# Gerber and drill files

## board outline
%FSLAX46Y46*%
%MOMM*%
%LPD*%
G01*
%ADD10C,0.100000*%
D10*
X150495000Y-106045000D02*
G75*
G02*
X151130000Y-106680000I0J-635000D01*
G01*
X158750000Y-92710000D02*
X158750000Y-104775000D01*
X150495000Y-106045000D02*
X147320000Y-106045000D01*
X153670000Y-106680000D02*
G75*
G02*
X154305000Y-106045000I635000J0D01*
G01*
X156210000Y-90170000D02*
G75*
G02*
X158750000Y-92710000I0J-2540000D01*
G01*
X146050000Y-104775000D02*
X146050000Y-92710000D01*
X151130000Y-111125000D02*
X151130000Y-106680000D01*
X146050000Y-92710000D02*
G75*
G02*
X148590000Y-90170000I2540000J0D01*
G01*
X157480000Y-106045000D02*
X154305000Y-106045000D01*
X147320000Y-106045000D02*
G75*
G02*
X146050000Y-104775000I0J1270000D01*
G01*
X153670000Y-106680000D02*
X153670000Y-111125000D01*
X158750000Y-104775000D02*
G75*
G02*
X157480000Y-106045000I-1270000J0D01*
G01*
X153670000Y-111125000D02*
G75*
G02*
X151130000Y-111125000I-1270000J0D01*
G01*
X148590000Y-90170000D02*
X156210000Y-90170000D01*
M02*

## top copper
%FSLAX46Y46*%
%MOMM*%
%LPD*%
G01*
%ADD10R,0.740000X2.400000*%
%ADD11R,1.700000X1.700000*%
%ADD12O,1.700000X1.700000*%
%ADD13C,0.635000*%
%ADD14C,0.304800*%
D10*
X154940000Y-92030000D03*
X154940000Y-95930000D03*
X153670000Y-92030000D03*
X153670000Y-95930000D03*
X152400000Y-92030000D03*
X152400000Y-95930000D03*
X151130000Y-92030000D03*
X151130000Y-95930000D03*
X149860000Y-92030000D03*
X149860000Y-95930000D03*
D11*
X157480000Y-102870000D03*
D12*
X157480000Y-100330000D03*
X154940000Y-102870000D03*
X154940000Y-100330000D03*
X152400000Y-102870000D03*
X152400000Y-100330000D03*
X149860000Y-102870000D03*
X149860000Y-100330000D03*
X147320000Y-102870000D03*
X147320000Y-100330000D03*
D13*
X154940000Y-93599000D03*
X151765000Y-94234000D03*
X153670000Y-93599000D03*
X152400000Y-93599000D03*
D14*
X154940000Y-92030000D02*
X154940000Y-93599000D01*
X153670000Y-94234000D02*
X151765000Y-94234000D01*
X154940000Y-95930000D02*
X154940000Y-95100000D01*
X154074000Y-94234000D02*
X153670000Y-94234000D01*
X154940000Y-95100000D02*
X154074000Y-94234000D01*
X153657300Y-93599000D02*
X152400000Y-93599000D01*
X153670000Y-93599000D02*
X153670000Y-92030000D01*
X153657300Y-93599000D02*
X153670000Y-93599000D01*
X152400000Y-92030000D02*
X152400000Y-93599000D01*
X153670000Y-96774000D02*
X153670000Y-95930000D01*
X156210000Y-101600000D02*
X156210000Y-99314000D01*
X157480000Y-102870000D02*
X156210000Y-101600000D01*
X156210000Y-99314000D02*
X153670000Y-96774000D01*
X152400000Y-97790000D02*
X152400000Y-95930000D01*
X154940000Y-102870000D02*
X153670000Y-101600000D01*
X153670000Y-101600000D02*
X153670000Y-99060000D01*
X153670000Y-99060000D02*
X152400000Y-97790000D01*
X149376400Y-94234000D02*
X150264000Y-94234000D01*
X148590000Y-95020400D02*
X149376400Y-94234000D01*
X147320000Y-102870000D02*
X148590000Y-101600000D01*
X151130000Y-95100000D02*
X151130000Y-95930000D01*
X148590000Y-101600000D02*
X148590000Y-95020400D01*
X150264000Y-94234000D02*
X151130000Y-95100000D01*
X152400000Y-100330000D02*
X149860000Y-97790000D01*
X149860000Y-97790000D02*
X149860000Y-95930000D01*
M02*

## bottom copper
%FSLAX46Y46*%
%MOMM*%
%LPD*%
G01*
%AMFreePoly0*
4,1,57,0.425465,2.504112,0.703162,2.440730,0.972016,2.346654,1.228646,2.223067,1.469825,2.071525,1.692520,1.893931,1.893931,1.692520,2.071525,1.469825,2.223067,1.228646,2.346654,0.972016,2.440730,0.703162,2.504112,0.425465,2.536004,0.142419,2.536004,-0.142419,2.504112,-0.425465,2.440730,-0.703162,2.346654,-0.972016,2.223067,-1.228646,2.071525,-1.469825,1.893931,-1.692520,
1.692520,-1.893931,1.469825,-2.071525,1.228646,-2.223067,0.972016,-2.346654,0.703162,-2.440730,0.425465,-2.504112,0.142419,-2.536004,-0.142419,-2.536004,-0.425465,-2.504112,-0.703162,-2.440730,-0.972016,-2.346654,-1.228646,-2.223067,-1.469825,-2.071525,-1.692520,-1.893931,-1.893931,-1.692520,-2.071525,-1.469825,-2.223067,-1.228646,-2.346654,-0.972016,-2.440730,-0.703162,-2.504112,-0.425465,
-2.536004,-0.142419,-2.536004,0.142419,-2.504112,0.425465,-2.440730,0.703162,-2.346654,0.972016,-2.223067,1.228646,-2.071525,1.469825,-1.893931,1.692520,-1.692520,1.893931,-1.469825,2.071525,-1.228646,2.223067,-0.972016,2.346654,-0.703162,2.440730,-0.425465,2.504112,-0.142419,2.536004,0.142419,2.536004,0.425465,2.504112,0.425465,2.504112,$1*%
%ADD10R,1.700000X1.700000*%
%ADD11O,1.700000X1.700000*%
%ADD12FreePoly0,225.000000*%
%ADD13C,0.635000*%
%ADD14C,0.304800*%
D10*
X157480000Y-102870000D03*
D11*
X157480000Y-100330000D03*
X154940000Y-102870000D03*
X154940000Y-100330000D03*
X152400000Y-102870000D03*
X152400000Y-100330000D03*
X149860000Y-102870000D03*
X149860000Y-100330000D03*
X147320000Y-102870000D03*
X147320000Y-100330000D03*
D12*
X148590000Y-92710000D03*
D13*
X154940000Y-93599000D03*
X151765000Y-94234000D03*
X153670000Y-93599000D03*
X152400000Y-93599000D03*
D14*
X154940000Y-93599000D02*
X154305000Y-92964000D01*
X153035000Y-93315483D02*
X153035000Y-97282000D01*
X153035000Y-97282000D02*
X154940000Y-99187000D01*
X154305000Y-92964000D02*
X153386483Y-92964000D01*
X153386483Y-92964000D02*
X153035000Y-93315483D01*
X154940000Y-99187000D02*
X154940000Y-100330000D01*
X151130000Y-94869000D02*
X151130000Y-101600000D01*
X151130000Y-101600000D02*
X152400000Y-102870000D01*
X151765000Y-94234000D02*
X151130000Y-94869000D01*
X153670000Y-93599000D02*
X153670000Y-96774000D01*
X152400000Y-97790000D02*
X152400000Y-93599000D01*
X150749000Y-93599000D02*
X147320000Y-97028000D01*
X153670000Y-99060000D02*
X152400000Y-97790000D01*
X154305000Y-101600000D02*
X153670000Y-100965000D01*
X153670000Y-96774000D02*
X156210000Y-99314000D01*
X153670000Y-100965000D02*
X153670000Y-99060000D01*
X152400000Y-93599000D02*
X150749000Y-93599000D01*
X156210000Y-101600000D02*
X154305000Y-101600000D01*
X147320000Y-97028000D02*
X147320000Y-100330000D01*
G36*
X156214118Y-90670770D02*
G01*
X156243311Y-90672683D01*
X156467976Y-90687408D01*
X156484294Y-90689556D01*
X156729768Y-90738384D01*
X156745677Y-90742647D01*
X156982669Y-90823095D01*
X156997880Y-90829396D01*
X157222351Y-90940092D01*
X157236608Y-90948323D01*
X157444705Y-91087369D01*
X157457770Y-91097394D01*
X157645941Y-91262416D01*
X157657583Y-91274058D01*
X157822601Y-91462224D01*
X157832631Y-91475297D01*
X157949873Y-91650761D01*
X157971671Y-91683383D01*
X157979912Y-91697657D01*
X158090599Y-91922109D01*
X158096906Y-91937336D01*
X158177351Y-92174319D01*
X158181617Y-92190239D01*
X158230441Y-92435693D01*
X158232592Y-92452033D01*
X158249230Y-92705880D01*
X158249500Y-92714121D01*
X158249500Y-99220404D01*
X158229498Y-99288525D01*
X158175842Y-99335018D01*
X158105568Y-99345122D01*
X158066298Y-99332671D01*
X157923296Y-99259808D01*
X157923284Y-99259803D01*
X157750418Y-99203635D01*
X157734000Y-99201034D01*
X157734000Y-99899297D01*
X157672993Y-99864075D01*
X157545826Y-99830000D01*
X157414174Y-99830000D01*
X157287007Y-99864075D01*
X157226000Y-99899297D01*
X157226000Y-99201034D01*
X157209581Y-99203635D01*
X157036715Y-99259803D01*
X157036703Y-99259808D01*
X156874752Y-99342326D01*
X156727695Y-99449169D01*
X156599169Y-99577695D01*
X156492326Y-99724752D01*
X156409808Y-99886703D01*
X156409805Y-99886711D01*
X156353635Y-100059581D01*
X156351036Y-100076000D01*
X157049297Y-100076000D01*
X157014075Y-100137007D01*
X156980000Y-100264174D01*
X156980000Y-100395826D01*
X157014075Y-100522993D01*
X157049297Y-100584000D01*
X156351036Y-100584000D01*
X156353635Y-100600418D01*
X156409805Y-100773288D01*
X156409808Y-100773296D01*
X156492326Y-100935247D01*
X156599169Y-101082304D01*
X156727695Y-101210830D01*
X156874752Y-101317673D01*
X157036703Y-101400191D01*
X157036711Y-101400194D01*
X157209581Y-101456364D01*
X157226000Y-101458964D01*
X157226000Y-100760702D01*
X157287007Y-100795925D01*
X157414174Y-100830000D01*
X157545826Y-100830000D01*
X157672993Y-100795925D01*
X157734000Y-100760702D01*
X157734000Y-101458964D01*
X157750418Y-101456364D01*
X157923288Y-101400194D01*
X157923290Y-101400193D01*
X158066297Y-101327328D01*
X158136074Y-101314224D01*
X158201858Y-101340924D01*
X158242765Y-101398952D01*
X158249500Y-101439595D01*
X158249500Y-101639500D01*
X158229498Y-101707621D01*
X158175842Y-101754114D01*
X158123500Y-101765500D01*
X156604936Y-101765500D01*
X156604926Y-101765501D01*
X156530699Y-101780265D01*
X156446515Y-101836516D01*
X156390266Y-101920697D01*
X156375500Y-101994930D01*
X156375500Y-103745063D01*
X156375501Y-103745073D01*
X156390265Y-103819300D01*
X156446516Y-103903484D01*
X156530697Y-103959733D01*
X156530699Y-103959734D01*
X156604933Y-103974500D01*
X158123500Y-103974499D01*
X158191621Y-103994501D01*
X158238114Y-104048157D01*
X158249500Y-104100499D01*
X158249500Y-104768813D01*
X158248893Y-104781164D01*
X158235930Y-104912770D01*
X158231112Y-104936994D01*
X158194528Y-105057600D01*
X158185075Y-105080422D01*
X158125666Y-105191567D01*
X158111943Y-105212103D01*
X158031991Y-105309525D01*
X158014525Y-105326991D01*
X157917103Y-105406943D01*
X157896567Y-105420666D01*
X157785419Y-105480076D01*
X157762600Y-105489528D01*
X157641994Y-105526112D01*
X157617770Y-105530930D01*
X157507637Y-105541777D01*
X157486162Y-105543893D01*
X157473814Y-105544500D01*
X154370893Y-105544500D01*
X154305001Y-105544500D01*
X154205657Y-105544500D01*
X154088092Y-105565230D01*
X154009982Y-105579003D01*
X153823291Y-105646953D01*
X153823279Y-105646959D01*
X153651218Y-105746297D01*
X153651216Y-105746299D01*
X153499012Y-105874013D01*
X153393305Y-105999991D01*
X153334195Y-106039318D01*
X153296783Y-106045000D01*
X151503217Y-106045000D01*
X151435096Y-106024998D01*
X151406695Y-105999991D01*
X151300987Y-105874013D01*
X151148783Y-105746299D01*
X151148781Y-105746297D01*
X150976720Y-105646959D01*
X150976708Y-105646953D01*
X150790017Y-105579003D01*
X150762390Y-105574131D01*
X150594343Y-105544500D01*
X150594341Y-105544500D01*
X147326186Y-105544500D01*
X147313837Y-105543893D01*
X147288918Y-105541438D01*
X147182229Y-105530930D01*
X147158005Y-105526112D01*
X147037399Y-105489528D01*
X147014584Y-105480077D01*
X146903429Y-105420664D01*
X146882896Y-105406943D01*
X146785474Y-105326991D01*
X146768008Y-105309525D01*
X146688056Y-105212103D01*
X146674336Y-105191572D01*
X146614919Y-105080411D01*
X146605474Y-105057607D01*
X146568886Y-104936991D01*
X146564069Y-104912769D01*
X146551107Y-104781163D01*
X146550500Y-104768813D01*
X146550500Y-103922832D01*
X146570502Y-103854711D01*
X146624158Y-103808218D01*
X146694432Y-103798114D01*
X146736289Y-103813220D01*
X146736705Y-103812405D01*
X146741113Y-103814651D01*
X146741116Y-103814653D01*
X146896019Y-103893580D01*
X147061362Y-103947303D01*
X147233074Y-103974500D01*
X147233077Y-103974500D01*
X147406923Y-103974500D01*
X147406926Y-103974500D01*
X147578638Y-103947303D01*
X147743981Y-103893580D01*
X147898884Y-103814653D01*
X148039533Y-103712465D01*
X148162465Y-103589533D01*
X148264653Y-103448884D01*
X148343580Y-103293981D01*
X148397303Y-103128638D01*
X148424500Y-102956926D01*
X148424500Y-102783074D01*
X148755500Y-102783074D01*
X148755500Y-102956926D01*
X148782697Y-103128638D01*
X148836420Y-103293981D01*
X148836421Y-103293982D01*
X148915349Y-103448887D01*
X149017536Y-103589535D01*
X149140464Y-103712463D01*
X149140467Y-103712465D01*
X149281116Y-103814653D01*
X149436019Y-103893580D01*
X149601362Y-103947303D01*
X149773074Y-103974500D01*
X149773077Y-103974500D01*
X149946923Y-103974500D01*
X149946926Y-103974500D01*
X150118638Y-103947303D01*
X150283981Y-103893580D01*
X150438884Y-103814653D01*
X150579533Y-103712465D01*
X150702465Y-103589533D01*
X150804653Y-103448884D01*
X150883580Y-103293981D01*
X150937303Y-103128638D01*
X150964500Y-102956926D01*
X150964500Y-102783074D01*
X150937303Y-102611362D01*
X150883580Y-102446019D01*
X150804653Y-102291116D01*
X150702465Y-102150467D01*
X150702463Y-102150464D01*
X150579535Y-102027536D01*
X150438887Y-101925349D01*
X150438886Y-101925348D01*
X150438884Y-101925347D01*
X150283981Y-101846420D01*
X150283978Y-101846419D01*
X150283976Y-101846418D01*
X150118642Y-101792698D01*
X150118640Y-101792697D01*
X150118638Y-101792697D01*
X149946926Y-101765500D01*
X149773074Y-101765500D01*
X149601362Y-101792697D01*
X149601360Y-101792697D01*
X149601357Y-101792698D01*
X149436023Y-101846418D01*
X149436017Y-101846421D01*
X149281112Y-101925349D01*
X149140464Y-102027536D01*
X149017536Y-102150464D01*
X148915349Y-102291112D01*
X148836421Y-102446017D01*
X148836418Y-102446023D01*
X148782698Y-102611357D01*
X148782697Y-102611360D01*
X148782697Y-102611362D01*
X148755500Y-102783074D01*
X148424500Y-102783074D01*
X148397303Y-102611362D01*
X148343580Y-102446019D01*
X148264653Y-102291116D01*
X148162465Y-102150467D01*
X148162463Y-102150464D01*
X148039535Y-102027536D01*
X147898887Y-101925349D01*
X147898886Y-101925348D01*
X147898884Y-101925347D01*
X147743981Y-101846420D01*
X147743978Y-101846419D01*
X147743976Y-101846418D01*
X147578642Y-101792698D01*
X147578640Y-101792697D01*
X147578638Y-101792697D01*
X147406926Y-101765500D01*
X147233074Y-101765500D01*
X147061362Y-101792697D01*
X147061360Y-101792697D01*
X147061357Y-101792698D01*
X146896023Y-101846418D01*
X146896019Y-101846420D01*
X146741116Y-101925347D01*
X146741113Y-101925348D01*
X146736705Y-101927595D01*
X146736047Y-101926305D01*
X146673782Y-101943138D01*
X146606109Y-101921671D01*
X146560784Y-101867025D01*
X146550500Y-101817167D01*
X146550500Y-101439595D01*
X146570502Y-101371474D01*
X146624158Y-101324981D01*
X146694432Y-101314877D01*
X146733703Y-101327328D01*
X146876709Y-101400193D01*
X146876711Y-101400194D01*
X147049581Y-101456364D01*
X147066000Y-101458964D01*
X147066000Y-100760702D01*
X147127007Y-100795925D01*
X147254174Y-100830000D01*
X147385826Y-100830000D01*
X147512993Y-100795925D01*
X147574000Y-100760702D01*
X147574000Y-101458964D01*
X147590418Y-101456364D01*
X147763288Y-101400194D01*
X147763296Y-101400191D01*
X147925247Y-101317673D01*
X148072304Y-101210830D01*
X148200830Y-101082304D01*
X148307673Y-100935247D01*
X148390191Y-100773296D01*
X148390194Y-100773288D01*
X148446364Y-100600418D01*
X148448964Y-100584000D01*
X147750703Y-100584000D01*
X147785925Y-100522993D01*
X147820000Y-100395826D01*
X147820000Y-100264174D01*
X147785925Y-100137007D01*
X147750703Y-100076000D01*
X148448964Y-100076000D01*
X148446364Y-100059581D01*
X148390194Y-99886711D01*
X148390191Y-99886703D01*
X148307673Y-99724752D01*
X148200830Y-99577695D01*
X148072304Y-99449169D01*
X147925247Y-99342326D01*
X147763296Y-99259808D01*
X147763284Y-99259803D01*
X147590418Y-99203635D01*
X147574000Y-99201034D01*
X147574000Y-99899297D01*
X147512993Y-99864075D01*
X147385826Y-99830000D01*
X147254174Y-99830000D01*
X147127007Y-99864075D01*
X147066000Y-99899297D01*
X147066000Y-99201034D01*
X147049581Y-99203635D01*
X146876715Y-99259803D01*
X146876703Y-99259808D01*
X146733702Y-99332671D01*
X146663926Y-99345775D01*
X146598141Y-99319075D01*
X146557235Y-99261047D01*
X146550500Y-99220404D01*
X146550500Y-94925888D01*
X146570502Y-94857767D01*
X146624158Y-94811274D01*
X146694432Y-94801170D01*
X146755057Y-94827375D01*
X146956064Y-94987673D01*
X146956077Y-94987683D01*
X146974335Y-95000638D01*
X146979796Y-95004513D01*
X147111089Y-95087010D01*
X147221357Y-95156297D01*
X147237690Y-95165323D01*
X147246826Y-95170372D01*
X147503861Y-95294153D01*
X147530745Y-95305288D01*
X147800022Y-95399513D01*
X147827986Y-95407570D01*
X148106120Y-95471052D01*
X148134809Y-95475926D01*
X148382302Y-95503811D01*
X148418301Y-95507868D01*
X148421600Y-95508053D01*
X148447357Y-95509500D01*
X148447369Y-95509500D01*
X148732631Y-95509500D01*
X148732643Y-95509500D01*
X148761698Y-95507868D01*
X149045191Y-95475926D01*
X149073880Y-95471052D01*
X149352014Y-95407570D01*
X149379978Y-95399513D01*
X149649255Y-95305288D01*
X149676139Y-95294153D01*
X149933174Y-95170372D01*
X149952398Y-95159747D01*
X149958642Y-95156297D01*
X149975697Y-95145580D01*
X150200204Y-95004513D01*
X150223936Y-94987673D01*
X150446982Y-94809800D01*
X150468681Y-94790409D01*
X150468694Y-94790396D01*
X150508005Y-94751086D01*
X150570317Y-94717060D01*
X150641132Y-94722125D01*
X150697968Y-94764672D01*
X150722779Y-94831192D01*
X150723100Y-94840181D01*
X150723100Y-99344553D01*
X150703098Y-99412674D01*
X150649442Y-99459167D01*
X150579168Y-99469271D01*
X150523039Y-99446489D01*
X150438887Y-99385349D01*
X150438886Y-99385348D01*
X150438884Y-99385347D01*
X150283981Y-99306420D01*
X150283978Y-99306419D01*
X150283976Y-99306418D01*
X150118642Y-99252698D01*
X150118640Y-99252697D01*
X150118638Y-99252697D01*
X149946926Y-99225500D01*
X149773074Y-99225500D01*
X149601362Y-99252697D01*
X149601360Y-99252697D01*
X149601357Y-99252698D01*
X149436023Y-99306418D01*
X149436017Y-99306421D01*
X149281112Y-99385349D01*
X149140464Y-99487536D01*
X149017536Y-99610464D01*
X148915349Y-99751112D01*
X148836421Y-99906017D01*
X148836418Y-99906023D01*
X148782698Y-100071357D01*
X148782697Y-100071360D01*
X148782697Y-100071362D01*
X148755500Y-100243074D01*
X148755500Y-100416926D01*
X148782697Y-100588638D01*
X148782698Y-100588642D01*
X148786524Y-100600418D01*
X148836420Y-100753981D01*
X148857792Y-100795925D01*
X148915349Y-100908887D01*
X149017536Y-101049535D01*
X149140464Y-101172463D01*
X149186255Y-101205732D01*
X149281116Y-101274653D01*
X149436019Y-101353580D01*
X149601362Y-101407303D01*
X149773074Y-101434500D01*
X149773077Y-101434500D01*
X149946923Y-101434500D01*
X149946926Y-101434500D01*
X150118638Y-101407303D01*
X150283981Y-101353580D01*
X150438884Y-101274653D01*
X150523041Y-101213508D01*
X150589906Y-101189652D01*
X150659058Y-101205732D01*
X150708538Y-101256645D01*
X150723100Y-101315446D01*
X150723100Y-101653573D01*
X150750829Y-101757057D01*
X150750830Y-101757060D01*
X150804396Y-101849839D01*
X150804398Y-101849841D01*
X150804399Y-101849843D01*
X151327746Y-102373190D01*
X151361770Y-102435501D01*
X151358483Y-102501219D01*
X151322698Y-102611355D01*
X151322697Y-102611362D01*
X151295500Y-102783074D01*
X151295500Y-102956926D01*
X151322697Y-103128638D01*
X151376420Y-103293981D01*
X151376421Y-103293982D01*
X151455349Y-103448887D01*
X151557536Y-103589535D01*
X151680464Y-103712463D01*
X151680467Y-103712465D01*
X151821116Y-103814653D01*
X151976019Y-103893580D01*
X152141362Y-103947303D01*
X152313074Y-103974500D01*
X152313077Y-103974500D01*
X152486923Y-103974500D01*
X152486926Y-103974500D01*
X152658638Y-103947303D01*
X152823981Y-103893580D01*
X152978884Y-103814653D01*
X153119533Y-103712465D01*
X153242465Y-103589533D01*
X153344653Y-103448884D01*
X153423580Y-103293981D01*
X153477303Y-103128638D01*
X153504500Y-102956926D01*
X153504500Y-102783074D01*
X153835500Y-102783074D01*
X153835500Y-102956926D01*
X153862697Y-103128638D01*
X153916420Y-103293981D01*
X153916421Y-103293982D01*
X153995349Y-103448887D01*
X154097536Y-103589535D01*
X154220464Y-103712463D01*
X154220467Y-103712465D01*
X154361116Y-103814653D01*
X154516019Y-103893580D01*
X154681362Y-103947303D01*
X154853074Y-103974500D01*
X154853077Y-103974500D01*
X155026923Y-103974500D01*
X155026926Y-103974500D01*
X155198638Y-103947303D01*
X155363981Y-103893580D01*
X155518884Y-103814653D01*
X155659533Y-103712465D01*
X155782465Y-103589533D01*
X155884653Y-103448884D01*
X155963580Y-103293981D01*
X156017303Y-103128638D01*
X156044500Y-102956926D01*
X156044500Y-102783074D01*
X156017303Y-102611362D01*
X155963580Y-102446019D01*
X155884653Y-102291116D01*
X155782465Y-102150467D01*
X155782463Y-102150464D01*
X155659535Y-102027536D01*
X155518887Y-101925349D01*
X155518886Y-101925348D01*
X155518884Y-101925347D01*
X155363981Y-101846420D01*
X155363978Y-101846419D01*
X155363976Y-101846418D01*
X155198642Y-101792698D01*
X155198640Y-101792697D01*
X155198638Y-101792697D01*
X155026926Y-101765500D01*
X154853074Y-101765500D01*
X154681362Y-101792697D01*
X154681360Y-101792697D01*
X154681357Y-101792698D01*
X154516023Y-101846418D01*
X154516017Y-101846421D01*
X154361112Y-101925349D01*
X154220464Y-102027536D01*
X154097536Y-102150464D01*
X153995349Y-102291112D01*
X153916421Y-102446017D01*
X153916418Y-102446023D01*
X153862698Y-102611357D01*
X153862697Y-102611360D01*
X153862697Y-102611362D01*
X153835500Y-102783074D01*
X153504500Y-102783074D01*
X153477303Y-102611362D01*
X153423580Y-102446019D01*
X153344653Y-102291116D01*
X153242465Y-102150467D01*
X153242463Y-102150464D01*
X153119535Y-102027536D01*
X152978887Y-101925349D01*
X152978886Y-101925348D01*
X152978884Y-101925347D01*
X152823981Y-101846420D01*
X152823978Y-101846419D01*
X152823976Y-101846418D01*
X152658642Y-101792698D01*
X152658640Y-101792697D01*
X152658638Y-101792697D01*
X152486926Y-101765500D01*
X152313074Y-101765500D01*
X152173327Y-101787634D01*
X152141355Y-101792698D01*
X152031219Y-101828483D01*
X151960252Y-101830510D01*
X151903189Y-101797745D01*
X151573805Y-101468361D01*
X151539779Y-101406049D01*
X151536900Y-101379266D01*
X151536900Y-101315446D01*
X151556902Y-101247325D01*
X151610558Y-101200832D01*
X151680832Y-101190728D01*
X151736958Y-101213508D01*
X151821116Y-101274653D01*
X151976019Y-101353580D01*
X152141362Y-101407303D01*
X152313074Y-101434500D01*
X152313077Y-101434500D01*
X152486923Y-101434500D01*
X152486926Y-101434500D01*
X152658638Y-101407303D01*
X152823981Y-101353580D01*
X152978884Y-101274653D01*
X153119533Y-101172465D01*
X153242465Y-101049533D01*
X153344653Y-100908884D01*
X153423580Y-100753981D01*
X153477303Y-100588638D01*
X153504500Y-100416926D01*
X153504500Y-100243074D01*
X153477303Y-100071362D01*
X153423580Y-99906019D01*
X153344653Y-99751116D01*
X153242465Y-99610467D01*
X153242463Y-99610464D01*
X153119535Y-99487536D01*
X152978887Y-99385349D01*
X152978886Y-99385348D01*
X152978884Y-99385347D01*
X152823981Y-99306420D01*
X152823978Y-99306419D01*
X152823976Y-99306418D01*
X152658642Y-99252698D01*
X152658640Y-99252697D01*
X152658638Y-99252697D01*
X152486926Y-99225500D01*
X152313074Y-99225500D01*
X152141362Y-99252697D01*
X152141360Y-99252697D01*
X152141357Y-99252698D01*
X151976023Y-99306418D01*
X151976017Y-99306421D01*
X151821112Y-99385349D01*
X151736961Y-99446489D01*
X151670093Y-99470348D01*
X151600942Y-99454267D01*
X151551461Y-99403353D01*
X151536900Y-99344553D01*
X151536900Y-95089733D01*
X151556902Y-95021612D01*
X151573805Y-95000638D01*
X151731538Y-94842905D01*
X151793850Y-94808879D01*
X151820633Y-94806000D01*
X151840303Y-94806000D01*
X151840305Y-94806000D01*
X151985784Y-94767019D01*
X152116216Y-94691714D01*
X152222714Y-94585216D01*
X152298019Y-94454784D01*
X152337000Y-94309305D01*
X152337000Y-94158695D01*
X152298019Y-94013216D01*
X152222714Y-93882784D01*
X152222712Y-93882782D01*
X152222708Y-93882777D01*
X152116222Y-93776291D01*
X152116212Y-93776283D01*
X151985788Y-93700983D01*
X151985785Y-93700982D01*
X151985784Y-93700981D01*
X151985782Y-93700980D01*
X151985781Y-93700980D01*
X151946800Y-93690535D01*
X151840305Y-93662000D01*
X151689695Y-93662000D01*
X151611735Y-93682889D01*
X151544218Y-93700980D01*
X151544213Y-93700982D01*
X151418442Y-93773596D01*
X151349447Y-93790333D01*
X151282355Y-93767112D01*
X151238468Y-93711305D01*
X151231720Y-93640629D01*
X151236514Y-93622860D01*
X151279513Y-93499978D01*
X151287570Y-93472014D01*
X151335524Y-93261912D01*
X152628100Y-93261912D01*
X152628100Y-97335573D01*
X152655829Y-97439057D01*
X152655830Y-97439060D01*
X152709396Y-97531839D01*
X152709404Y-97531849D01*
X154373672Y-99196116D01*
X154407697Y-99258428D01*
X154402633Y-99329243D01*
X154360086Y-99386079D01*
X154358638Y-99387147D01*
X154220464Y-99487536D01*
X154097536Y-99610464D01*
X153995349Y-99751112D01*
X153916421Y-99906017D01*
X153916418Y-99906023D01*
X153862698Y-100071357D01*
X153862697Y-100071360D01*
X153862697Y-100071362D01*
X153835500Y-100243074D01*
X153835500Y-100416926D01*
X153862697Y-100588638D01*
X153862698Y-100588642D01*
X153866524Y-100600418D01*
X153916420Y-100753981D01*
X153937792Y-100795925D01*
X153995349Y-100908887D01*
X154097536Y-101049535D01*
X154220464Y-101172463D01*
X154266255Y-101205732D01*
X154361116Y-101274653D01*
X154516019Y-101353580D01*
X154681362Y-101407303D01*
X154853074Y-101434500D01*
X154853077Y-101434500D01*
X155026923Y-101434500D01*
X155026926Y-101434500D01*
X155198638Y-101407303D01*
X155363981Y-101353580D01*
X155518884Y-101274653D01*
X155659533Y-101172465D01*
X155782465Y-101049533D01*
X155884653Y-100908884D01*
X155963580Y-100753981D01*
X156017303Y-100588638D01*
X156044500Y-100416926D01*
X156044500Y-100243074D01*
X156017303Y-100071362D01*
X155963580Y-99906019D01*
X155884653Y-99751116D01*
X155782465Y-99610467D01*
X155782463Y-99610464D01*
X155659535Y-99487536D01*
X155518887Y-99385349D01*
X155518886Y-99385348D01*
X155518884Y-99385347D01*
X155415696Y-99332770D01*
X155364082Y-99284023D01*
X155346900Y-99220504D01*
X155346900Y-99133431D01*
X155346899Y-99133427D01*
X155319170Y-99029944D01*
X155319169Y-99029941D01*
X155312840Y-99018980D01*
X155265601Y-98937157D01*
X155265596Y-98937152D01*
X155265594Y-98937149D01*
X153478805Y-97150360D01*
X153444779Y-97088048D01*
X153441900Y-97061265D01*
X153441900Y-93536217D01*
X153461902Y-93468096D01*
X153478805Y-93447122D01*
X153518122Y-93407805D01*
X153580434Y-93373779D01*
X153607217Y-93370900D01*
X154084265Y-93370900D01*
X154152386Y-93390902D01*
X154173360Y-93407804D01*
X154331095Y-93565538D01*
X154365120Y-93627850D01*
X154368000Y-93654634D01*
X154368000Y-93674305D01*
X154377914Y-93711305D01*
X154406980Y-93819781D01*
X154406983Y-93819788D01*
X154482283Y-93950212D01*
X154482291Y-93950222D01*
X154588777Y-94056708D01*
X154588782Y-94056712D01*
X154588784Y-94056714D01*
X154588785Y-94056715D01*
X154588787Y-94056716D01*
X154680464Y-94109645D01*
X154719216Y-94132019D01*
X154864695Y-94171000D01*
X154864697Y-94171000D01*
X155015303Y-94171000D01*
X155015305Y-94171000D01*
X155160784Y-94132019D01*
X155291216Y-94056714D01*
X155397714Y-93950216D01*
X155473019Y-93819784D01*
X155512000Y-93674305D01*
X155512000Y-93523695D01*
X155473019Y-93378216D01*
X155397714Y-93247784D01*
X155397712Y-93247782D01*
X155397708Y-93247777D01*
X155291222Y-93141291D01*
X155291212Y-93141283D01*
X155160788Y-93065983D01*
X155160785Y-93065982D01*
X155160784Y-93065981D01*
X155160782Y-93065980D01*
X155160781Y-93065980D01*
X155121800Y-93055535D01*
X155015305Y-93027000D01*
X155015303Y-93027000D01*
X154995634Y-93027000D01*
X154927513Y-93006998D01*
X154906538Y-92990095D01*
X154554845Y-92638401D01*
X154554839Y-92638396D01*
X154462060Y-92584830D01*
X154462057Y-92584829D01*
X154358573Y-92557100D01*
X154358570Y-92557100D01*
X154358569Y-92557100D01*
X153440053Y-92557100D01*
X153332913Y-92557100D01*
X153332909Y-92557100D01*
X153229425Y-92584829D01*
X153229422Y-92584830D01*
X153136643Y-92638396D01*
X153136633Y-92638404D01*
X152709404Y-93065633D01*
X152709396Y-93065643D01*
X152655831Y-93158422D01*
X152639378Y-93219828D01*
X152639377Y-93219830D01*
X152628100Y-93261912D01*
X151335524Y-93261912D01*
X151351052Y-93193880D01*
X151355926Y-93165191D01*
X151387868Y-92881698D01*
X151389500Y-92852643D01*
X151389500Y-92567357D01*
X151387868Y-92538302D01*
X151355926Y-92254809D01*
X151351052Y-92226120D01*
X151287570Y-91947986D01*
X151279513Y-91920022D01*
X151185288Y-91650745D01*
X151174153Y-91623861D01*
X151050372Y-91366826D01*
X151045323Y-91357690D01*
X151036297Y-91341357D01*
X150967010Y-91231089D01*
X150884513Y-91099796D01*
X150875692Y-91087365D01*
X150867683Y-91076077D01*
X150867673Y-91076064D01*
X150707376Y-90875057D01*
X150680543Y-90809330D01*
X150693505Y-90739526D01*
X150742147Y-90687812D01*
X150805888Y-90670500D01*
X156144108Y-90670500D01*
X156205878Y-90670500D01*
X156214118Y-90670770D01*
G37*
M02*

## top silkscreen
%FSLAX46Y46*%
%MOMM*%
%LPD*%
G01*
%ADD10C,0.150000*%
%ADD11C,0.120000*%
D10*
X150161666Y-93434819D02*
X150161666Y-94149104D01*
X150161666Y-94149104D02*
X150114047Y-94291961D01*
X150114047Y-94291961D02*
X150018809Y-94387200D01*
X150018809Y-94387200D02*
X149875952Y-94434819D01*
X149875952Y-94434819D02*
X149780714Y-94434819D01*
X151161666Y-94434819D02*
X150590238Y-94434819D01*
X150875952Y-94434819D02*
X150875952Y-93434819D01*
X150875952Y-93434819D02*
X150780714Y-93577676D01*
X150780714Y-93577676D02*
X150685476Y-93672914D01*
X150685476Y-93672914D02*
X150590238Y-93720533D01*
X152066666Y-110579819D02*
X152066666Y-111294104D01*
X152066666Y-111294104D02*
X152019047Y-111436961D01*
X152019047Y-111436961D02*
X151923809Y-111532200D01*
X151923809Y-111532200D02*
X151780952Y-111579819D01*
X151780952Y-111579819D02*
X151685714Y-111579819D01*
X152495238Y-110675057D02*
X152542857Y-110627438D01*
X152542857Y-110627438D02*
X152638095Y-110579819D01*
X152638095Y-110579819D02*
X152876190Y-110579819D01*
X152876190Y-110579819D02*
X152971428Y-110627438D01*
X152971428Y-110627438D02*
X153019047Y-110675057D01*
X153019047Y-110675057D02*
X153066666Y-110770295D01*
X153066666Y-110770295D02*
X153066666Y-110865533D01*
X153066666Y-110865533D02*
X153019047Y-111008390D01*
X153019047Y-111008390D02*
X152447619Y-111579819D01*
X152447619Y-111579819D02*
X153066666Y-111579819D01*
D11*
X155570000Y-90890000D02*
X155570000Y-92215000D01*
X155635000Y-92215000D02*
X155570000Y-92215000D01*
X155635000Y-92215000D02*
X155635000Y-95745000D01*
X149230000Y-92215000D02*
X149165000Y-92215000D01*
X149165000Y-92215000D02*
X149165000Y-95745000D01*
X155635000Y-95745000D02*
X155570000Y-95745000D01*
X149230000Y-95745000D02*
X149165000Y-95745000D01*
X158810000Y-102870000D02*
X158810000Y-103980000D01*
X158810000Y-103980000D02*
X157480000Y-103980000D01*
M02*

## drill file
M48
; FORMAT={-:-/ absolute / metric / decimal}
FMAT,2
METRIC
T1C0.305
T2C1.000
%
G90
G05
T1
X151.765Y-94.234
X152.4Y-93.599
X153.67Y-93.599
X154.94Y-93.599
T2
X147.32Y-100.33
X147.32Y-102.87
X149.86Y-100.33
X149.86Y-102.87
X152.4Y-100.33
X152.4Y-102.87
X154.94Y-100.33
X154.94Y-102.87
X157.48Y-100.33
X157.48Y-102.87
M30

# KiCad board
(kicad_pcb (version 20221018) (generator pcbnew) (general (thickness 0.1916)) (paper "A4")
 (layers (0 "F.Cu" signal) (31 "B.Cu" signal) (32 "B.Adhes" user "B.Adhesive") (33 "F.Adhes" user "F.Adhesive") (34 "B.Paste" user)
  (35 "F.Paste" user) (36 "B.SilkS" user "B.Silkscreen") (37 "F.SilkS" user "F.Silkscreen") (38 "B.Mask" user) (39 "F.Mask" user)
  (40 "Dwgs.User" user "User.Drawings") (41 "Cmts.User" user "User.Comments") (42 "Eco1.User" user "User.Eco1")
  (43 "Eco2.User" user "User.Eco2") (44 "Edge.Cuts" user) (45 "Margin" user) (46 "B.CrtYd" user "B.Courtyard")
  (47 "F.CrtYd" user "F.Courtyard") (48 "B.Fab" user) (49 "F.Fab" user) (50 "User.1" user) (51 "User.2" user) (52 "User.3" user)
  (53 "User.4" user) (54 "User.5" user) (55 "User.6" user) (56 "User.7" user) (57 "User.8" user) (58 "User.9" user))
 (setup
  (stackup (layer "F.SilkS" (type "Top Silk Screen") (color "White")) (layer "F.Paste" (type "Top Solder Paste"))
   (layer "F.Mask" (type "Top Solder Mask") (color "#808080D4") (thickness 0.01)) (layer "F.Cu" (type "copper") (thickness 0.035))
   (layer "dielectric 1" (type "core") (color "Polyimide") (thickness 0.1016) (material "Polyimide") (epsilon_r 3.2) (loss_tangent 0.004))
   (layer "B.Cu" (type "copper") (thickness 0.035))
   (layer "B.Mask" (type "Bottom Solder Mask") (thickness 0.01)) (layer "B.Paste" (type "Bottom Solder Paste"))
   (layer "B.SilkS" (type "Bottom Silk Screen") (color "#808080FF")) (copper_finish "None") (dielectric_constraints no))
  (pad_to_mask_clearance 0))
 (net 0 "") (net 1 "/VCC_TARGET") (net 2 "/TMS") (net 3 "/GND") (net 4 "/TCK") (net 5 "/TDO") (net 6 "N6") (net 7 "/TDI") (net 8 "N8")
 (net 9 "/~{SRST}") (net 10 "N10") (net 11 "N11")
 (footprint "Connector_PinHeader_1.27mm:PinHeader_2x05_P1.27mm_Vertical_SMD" (layer "F.Cu") (at 152.4 93.98 -90)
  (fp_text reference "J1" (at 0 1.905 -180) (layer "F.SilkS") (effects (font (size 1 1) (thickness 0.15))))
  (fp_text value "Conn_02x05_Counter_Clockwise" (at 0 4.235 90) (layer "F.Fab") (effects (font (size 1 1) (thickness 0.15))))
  (fp_line (start -3.09 -3.17) (end -1.765 -3.17) (stroke (width 0.12) (type solid)) (layer "F.SilkS"))
  (fp_line (start -1.765 -3.235) (end -1.765 -3.17) (stroke (width 0.12) (type solid)) (layer "F.SilkS"))
  (fp_line (start -1.765 -3.235) (end 1.765 -3.235) (stroke (width 0.12) (type solid)) (layer "F.SilkS"))
  (fp_line (start -1.765 3.17) (end -1.765 3.235) (stroke (width 0.12) (type solid)) (layer "F.SilkS"))
  (fp_line (start -1.765 3.235) (end 1.765 3.235) (stroke (width 0.12) (type solid)) (layer "F.SilkS"))
  (fp_line (start 1.765 -3.235) (end 1.765 -3.17) (stroke (width 0.12) (type solid)) (layer "F.SilkS"))
  (fp_line (start 1.765 3.17) (end 1.765 3.235) (stroke (width 0.12) (type solid)) (layer "F.SilkS"))
  (pad "1" smd rect (at -1.95 -2.54 270) (size 2.4 0.74) (layers "F.Cu" "F.Paste" "F.Mask") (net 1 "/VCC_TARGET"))
  (pad "2" smd rect (at 1.95 -2.54 270) (size 2.4 0.74) (layers "F.Cu" "F.Paste" "F.Mask") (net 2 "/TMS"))
  (pad "3" smd rect (at -1.95 -1.27 270) (size 2.4 0.74) (layers "F.Cu" "F.Paste" "F.Mask") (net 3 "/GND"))
  (pad "4" smd rect (at 1.95 -1.27 270) (size 2.4 0.74) (layers "F.Cu" "F.Paste" "F.Mask") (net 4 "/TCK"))
  (pad "5" smd rect (at -1.95 0 270) (size 2.4 0.74) (layers "F.Cu" "F.Paste" "F.Mask") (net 3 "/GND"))
  (pad "6" smd rect (at 1.95 0 270) (size 2.4 0.74) (layers "F.Cu" "F.Paste" "F.Mask") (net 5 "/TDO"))
  (pad "7" smd rect (at -1.95 1.27 270) (size 2.4 0.74) (layers "F.Cu" "F.Paste" "F.Mask") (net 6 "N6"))
  (pad "8" smd rect (at 1.95 1.27 270) (size 2.4 0.74) (layers "F.Cu" "F.Paste" "F.Mask") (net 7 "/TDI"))
  (pad "9" smd rect (at -1.95 2.54 270) (size 2.4 0.74) (layers "F.Cu" "F.Paste" "F.Mask") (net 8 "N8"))
  (pad "10" smd rect (at 1.95 2.54 270) (size 2.4 0.74) (layers "F.Cu" "F.Paste" "F.Mask") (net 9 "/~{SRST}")))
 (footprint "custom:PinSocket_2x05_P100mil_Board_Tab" (layer "F.Cu") (at 157.48 102.87 -90)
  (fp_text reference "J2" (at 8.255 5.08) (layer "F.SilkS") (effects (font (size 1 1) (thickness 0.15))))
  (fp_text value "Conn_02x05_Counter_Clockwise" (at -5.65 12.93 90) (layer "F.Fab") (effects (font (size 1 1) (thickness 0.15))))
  (fp_line (start 0 -1.33) (end 1.11 -1.33) (stroke (width 0.12) (type solid)) (layer "F.SilkS"))
  (fp_line (start 1.11 -1.33) (end 1.11 0) (stroke (width 0.12) (type solid)) (layer "F.SilkS"))
  (pad "1" thru_hole rect (at 0 0 270) (size 1.7 1.7) (drill 1) (layers "*.Cu" "*.Mask") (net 4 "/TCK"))
  (pad "2" thru_hole oval (at -2.54 0 270) (size 1.7 1.7) (drill 1) (layers "*.Cu" "*.Mask") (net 3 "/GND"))
  (pad "3" thru_hole oval (at 0 2.54 270) (size 1.7 1.7) (drill 1) (layers "*.Cu" "*.Mask") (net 5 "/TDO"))
  (pad "4" thru_hole oval (at -2.54 2.54 270) (size 1.7 1.7) (drill 1) (layers "*.Cu" "*.Mask") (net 1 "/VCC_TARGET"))
  (pad "5" thru_hole oval (at 0 5.08 270) (size 1.7 1.7) (drill 1) (layers "*.Cu" "*.Mask") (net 2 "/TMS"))
  (pad "6" thru_hole oval (at -2.54 5.08 270) (size 1.7 1.7) (drill 1) (layers "*.Cu" "*.Mask") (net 9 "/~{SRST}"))
  (pad "7" thru_hole oval (at 0 7.62 270) (size 1.7 1.7) (drill 1) (layers "*.Cu" "*.Mask") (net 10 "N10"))
  (pad "8" thru_hole oval (at -2.54 7.62 270) (size 1.7 1.7) (drill 1) (layers "*.Cu" "*.Mask") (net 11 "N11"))
  (pad "9" thru_hole oval (at 0 10.16 270) (size 1.7 1.7) (drill 1) (layers "*.Cu" "*.Mask") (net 7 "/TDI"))
  (pad "10" thru_hole oval (at -2.54 10.16 270) (size 1.7 1.7) (drill 1) (layers "*.Cu" "*.Mask") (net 3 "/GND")))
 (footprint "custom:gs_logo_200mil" (layer "B.Cu") (at 148.59 92.71 -135)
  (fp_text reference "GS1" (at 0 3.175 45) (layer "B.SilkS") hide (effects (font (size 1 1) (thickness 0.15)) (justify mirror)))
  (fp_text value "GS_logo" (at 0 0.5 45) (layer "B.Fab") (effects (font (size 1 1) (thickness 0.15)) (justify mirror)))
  (pad "1" smd custom (at 0 0 225) (size 5.08 5.08) (layers "B.Cu") (zone_connect 0) (options (clearance outline) (anchor circle))
   (primitives)))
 (gr_arc (start 150.495 106.045) (mid 150.944013 106.230987) (end 151.13 106.68) (stroke (width 0.1) (type default)) (layer "Edge.Cuts"))
 (gr_line (start 158.75 92.71) (end 158.75 104.775) (stroke (width 0.1) (type default)) (layer "Edge.Cuts"))
 (gr_line (start 150.495 106.045) (end 147.32 106.045) (stroke (width 0.1) (type default)) (layer "Edge.Cuts"))
 (gr_arc (start 153.67 106.68) (mid 153.855987 106.230987) (end 154.305 106.045) (stroke (width 0.1) (type default)) (layer "Edge.Cuts"))
 (gr_arc (start 156.21 90.17) (mid 158.006051 90.913949) (end 158.75 92.71) (stroke (width 0.1) (type default)) (layer "Edge.Cuts"))
 (gr_line (start 146.05 104.775) (end 146.05 92.71) (stroke (width 0.1) (type default)) (layer "Edge.Cuts"))
 (gr_line (start 151.13 111.125) (end 151.13 106.68) (stroke (width 0.1) (type default)) (layer "Edge.Cuts"))
 (gr_arc (start 146.05 92.71) (mid 146.793949 90.913949) (end 148.59 90.17) (stroke (width 0.1) (type default)) (layer "Edge.Cuts"))
 (gr_line (start 157.48 106.045) (end 154.305 106.045) (stroke (width 0.1) (type default)) (layer "Edge.Cuts"))
 (gr_arc (start 147.32 106.045) (mid 146.421974 105.673026) (end 146.05 104.775) (stroke (width 0.1) (type default)) (layer "Edge.Cuts"))
 (gr_line (start 153.67 106.68) (end 153.67 111.125) (stroke (width 0.1) (type default)) (layer "Edge.Cuts"))
 (gr_arc (start 158.75 104.775) (mid 158.378026 105.673026) (end 157.48 106.045) (stroke (width 0.1) (type default)) (layer "Edge.Cuts"))
 (gr_arc (start 153.67 111.125) (mid 152.4 112.395) (end 151.13 111.125) (stroke (width 0.1) (type default)) (layer "Edge.Cuts"))
 (gr_line (start 148.59 90.17) (end 156.21 90.17) (stroke (width 0.1) (type default)) (layer "Edge.Cuts"))
 (segment (start 154.94 92.03) (end 154.94 93.599) (width 0.3048) (layer "F.Cu") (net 1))
 (via (at 154.94 93.599) (size 0.635) (drill 0.3048) (layers "F.Cu" "B.Cu") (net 1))
 (segment (start 154.94 93.599) (end 154.305 92.964) (width 0.3048) (layer "B.Cu") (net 1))
 (segment (start 153.035 93.315483) (end 153.035 97.282) (width 0.3048) (layer "B.Cu") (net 1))
 (segment (start 153.035 97.282) (end 154.94 99.187) (width 0.3048) (layer "B.Cu") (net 1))
 (segment (start 154.305 92.964) (end 153.386483 92.964) (width 0.3048) (layer "B.Cu") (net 1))
 (segment (start 153.386483 92.964) (end 153.035 93.315483) (width 0.3048) (layer "B.Cu") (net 1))
 (segment (start 154.94 99.187) (end 154.94 100.33) (width 0.3048) (layer "B.Cu") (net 1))
 (segment (start 153.67 94.234) (end 151.765 94.234) (width 0.3048) (layer "F.Cu") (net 2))
 (segment (start 154.94 95.93) (end 154.94 95.1) (width 0.3048) (layer "F.Cu") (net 2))
 (segment (start 154.074 94.234) (end 153.67 94.234) (width 0.3048) (layer "F.Cu") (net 2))
 (segment (start 154.94 95.1) (end 154.074 94.234) (width 0.3048) (layer "F.Cu") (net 2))
 (via (at 151.765 94.234) (size 0.635) (drill 0.3048) (layers "F.Cu" "B.Cu") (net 2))
 (segment (start 151.13 94.869) (end 151.13 101.6) (width 0.3048) (layer "B.Cu") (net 2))
 (segment (start 151.13 101.6) (end 152.4 102.87) (width 0.3048) (layer "B.Cu") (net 2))
 (segment (start 151.765 94.234) (end 151.13 94.869) (width 0.3048) (layer "B.Cu") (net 2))
 (segment (start 153.6573 93.599) (end 152.4 93.599) (width 0.3048) (layer "F.Cu") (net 3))
 (segment (start 153.67 93.599) (end 153.67 92.03) (width 0.3048) (layer "F.Cu") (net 3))
 (segment (start 153.6573 93.599) (end 153.67 93.599) (width 0.3048) (layer "F.Cu") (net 3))
 (segment (start 152.4 92.03) (end 152.4 93.599) (width 0.3048) (layer "F.Cu") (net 3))
 (via (at 153.67 93.599) (size 0.635) (drill 0.3048) (layers "F.Cu" "B.Cu") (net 3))
 (via (at 152.4 93.599) (size 0.635) (drill 0.3048) (layers "F.Cu" "B.Cu") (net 3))
 (segment (start 153.67 93.599) (end 153.67 96.774) (width 0.3048) (layer "B.Cu") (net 3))
 (segment (start 152.4 97.79) (end 152.4 93.599) (width 0.3048) (layer "B.Cu") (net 3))
 (segment (start 150.749 93.599) (end 147.32 97.028) (width 0.3048) (layer "B.Cu") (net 3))
 (segment (start 153.67 99.06) (end 152.4 97.79) (width 0.3048) (layer "B.Cu") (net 3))
 (segment (start 154.305 101.6) (end 153.67 100.965) (width 0.3048) (layer "B.Cu") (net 3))
 (segment (start 153.67 96.774) (end 156.21 99.314) (width 0.3048) (layer "B.Cu") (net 3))
 (segment (start 153.67 100.965) (end 153.67 99.06) (width 0.3048) (layer "B.Cu") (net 3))
 (segment (start 152.4 93.599) (end 150.749 93.599) (width 0.3048) (layer "B.Cu") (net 3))
 (segment (start 156.21 101.6) (end 154.305 101.6) (width 0.3048) (layer "B.Cu") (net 3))
 (segment (start 147.32 97.028) (end 147.32 100.33) (width 0.3048) (layer "B.Cu") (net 3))
 (segment (start 153.67 96.774) (end 153.67 95.93) (width 0.3048) (layer "F.Cu") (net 4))
 (segment (start 156.21 101.6) (end 156.21 99.314) (width 0.3048) (layer "F.Cu") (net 4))
 (segment (start 157.48 102.87) (end 156.21 101.6) (width 0.3048) (layer "F.Cu") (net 4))
 (segment (start 156.21 99.314) (end 153.67 96.774) (width 0.3048) (layer "F.Cu") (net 4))
 (segment (start 152.4 97.79) (end 152.4 95.93) (width 0.3048) (layer "F.Cu") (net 5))
 (segment (start 154.94 102.87) (end 153.67 101.6) (width 0.3048) (layer "F.Cu") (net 5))
 (segment (start 153.67 101.6) (end 153.67 99.06) (width 0.3048) (layer "F.Cu") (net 5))
 (segment (start 153.67 99.06) (end 152.4 97.79) (width 0.3048) (layer "F.Cu") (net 5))
 (segment (start 149.3764 94.234) (end 150.264 94.234) (width 0.3048) (layer "F.Cu") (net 7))
 (segment (start 148.59 95.0204) (end 149.3764 94.234) (width 0.3048) (layer "F.Cu") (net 7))
 (segment (start 147.32 102.87) (end 148.59 101.6) (width 0.3048) (layer "F.Cu") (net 7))
 (segment (start 151.13 95.1) (end 151.13 95.93) (width 0.3048) (layer "F.Cu") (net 7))
 (segment (start 148.59 101.6) (end 148.59 95.0204) (width 0.3048) (layer "F.Cu") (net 7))
 (segment (start 150.264 94.234) (end 151.13 95.1) (width 0.3048) (layer "F.Cu") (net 7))
 (segment (start 152.4 100.33) (end 149.86 97.79) (width 0.3048) (layer "F.Cu") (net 9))
 (segment (start 149.86 97.79) (end 149.86 95.93) (width 0.3048) (layer "F.Cu") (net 9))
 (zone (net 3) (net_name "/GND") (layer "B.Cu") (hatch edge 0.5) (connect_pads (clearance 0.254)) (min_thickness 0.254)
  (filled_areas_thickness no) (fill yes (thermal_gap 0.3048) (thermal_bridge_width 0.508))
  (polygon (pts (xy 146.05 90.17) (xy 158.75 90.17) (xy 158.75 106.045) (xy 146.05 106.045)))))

